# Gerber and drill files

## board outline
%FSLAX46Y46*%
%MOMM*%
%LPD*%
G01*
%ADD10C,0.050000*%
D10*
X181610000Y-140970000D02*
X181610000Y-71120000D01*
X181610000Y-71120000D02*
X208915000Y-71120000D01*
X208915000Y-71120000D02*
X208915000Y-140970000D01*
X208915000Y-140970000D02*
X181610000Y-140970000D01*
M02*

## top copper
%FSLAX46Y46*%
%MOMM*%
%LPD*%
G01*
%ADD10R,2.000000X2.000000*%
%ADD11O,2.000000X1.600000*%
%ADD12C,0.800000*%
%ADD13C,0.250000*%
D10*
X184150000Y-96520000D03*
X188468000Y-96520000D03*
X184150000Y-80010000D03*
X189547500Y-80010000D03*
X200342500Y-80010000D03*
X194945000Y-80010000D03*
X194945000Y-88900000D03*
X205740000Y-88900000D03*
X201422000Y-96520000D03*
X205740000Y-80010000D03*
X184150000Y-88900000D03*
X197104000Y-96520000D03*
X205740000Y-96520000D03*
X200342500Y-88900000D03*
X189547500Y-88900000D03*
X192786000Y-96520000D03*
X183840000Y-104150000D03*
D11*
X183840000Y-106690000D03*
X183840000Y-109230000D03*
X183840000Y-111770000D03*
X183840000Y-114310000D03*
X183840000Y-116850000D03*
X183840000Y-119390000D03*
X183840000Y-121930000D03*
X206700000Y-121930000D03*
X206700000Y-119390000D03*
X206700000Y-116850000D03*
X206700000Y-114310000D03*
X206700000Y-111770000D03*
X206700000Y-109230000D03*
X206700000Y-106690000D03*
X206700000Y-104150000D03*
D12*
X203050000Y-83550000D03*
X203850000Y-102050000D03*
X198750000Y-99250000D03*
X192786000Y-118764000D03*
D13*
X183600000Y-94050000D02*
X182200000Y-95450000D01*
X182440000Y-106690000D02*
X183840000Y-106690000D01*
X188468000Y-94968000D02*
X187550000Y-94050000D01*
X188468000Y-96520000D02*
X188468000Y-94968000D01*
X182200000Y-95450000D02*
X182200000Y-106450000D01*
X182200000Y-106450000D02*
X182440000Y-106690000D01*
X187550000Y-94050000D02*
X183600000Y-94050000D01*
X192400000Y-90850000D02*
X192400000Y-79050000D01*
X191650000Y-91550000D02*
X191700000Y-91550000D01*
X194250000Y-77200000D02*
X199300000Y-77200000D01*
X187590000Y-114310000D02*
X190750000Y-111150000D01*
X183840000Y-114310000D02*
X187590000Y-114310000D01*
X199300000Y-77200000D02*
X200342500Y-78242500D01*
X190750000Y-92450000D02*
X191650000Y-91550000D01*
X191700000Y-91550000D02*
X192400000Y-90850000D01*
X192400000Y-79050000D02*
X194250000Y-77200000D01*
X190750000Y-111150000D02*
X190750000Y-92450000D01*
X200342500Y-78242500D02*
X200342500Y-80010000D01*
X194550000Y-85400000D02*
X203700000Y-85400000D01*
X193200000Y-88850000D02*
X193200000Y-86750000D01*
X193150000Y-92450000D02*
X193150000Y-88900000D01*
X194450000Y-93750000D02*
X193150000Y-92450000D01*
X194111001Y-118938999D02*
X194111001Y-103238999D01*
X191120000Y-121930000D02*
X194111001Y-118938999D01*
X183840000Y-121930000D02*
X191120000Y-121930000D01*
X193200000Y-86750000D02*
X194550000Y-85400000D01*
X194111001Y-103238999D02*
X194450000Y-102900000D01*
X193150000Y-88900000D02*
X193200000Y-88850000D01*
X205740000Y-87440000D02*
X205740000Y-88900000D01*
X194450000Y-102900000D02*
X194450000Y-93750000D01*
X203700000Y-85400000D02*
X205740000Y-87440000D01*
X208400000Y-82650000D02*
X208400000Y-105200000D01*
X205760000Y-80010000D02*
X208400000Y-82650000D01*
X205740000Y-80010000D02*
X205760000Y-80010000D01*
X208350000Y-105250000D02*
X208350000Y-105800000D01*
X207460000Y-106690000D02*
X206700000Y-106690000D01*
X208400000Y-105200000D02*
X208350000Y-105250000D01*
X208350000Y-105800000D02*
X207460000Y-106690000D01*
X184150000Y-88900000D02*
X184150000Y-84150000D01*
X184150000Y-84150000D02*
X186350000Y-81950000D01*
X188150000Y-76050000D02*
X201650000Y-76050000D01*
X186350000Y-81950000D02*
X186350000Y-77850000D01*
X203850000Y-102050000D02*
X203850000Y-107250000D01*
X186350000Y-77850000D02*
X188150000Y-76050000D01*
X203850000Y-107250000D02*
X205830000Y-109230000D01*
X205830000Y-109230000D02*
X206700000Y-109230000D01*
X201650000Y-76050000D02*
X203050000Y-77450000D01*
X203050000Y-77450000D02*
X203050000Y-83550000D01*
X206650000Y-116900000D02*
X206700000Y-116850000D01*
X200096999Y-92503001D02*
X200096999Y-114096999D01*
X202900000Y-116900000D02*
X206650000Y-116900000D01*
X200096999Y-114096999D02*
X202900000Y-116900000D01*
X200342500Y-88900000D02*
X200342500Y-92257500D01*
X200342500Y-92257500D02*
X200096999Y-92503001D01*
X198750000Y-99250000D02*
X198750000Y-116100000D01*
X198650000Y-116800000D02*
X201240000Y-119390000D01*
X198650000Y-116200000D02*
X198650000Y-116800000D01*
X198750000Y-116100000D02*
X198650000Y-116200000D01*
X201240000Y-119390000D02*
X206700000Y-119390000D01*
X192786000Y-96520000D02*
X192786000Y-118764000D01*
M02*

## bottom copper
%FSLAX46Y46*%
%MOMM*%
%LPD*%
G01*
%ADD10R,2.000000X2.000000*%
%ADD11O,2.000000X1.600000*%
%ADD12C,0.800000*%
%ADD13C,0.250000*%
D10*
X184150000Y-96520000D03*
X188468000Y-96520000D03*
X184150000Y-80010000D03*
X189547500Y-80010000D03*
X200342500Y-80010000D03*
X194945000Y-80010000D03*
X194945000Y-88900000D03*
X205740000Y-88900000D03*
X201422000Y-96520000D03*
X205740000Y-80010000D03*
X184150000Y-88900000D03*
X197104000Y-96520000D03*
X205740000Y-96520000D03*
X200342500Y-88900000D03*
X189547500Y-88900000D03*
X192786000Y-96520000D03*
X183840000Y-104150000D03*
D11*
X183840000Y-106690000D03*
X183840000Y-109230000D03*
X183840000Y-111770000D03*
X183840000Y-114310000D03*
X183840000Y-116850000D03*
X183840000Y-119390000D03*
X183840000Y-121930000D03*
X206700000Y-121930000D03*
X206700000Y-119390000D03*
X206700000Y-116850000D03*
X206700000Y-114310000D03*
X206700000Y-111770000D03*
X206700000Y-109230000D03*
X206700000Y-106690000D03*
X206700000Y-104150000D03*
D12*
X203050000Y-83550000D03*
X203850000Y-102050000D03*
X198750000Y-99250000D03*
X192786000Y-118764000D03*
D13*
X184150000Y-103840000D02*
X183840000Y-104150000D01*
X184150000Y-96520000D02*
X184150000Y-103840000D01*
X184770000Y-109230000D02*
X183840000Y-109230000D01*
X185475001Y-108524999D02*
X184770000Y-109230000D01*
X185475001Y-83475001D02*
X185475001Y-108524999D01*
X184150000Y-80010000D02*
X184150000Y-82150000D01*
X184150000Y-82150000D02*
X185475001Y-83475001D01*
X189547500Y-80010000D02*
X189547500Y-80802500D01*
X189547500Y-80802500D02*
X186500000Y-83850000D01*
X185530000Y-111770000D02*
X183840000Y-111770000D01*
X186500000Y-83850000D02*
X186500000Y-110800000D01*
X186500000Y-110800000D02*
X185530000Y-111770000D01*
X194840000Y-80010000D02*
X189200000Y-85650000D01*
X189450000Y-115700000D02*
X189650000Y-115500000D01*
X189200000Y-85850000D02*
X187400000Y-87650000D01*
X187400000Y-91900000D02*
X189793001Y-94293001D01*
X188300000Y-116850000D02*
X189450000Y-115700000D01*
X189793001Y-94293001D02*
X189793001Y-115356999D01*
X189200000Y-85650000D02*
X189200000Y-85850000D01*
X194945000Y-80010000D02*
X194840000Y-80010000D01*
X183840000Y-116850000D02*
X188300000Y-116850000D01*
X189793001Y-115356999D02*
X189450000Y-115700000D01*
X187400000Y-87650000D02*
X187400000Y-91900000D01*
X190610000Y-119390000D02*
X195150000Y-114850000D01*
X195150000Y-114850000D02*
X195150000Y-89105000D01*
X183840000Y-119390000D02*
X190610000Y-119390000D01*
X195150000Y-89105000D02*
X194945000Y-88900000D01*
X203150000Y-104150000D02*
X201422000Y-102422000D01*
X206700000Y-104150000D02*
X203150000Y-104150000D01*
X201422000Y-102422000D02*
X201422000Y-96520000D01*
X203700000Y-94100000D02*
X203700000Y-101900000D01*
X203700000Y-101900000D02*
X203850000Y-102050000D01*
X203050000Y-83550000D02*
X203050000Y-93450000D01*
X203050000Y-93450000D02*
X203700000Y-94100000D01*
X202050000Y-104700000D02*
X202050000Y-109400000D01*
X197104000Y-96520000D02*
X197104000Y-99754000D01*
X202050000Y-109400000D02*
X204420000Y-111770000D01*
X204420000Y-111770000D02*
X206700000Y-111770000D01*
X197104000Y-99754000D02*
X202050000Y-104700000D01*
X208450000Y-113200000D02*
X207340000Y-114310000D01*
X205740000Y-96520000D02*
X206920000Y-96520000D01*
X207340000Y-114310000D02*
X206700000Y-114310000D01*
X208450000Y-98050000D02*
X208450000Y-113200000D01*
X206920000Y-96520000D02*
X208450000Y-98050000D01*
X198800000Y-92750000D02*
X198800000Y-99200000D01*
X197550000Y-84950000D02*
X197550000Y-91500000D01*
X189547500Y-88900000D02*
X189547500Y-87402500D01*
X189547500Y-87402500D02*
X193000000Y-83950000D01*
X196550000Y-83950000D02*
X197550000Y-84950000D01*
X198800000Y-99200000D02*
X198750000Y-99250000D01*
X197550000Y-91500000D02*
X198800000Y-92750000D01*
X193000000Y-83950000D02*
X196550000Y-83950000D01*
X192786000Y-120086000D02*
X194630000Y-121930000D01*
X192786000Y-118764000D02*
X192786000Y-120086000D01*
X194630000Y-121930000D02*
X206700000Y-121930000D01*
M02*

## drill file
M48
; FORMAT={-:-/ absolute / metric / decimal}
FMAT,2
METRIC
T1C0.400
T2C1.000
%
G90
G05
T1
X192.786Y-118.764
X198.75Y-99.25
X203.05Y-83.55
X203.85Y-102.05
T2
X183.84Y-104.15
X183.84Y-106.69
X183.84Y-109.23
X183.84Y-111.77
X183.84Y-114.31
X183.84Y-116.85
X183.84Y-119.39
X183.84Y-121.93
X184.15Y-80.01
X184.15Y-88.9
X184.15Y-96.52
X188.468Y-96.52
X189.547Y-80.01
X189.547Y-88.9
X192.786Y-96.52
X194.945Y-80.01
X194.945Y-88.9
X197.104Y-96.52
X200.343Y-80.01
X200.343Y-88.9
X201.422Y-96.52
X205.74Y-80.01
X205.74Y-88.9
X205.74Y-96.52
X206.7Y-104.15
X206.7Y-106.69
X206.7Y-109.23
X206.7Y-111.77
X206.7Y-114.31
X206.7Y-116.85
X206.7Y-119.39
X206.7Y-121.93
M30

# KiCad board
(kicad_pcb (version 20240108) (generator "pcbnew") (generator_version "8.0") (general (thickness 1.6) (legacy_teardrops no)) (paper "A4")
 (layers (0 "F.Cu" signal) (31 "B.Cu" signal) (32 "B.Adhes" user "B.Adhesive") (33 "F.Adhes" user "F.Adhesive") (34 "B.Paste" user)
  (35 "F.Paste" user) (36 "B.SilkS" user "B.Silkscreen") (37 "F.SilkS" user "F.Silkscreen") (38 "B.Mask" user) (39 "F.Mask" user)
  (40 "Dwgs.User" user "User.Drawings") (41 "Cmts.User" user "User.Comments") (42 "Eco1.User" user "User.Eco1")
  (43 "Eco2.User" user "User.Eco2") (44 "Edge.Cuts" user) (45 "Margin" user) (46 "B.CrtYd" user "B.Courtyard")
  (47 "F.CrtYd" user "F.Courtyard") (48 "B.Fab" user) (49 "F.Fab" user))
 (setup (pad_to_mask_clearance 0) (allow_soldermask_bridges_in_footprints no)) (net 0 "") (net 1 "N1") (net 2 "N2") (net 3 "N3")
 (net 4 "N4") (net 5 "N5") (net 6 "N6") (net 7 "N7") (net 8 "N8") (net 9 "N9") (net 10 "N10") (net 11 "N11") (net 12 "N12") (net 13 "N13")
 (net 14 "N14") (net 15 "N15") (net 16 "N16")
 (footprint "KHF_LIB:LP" (layer "F.Cu") (at 184.15 96.52)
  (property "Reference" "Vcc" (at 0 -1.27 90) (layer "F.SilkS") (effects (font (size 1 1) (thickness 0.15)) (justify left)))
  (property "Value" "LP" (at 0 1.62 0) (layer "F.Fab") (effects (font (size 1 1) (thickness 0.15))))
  (pad "1" thru_hole rect (at 0 0) (size 2 2) (drill 1) (layers "*.Cu" "*.Mask") (remove_unused_layers no) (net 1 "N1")))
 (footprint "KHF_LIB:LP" (layer "F.Cu") (at 188.468 96.52)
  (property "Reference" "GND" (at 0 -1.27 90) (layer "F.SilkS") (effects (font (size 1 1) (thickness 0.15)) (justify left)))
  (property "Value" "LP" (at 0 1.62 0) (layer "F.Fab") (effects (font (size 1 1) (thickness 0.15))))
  (pad "1" thru_hole rect (at 0 0) (size 2 2) (drill 1) (layers "*.Cu" "*.Mask") (remove_unused_layers no) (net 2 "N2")))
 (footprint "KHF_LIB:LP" (layer "F.Cu") (at 184.15 80.01)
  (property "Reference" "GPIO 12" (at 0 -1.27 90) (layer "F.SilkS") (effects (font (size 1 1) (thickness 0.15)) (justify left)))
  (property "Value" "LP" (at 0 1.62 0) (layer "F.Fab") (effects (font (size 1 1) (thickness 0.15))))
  (pad "1" thru_hole rect (at 0 0) (size 2 2) (drill 1) (layers "*.Cu" "*.Mask") (remove_unused_layers no) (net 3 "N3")))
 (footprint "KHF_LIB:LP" (layer "F.Cu") (at 189.5475 80.01)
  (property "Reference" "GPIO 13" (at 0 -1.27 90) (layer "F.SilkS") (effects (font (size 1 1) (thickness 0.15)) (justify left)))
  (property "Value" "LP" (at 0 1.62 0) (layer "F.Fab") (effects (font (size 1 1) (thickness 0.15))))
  (pad "1" thru_hole rect (at 0 0) (size 2 2) (drill 1) (layers "*.Cu" "*.Mask") (remove_unused_layers no) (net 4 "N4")))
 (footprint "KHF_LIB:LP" (layer "F.Cu") (at 200.3425 80.01)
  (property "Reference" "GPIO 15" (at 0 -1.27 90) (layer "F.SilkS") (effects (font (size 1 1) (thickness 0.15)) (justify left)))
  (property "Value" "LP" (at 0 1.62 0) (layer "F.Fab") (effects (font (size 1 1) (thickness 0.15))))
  (pad "1" thru_hole rect (at 0 0) (size 2 2) (drill 1) (layers "*.Cu" "*.Mask") (remove_unused_layers no) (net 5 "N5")))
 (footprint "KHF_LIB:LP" (layer "F.Cu") (at 194.945 80.01)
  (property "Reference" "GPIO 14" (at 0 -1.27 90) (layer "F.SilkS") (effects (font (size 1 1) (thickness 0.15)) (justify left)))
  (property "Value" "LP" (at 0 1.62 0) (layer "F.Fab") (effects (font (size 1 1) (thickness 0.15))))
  (pad "1" thru_hole rect (at 0 0) (size 2 2) (drill 1) (layers "*.Cu" "*.Mask") (remove_unused_layers no) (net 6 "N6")))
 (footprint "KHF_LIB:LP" (layer "F.Cu") (at 194.945 88.9)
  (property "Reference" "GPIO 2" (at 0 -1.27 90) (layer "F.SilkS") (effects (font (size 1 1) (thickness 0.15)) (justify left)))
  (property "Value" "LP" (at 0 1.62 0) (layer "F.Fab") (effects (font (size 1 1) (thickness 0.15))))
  (pad "1" thru_hole rect (at 0 0) (size 2 2) (drill 1) (layers "*.Cu" "*.Mask") (remove_unused_layers no) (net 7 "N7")))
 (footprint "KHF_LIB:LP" (layer "F.Cu") (at 205.74 88.9)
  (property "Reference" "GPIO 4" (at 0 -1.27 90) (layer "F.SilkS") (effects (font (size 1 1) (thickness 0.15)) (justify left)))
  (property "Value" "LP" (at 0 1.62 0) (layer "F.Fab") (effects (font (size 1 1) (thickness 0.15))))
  (pad "1" thru_hole rect (at 0 0) (size 2 2) (drill 1) (layers "*.Cu" "*.Mask") (remove_unused_layers no) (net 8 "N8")))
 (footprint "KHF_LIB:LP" (layer "F.Cu") (at 201.422 96.52)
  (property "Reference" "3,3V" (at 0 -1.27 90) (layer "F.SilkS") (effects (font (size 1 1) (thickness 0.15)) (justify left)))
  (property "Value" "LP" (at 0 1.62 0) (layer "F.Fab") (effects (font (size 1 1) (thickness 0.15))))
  (pad "1" thru_hole rect (at 0 0) (size 2 2) (drill 1) (layers "*.Cu" "*.Mask") (remove_unused_layers no) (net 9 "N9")))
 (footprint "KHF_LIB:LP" (layer "F.Cu") (at 205.74 80.01)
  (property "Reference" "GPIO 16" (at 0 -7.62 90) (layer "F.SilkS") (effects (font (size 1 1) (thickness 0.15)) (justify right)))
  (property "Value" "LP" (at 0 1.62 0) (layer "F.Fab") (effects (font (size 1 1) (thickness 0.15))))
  (pad "1" thru_hole rect (at 0 0) (size 2 2) (drill 1) (layers "*.Cu" "*.Mask") (remove_unused_layers no) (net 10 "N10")))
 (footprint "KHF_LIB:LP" (layer "F.Cu") (at 184.15 88.9)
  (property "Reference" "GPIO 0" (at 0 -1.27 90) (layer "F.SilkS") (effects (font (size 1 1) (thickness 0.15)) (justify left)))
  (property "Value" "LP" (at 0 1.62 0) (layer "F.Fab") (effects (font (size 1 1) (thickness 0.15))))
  (pad "1" thru_hole rect (at 0 0) (size 2 2) (drill 1) (layers "*.Cu" "*.Mask") (remove_unused_layers no) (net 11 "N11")))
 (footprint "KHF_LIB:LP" (layer "F.Cu") (at 197.104 96.52)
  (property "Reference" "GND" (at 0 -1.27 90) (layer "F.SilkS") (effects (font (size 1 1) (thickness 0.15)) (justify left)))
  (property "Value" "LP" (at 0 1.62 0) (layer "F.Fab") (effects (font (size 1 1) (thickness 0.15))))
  (pad "1" thru_hole rect (at 0 0) (size 2 2) (drill 1) (layers "*.Cu" "*.Mask") (remove_unused_layers no) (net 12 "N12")))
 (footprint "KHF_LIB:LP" (layer "F.Cu") (at 205.74 96.52)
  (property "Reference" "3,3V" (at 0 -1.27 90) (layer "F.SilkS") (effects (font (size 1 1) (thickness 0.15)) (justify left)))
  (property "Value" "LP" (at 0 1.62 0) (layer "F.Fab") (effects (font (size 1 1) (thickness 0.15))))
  (pad "1" thru_hole rect (at 0 0) (size 2 2) (drill 1) (layers "*.Cu" "*.Mask") (remove_unused_layers no) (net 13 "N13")))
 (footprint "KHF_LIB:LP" (layer "F.Cu") (at 200.3425 88.9)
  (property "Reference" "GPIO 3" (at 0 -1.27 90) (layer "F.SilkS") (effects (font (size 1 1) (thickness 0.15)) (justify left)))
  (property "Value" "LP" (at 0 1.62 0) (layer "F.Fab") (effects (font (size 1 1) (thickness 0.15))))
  (pad "1" thru_hole rect (at 0 0) (size 2 2) (drill 1) (layers "*.Cu" "*.Mask") (remove_unused_layers no) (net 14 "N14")))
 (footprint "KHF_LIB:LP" (layer "F.Cu") (at 189.5475 88.9)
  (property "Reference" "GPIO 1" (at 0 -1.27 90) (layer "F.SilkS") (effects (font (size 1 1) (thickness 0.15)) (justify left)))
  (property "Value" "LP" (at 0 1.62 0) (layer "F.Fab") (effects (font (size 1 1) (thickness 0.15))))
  (pad "1" thru_hole rect (at 0 0) (size 2 2) (drill 1) (layers "*.Cu" "*.Mask") (remove_unused_layers no) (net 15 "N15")))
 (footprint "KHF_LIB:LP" (layer "F.Cu") (at 192.786 96.52)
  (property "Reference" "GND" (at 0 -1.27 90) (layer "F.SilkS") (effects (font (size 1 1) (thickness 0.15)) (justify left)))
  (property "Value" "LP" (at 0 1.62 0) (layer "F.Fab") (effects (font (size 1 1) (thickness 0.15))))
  (pad "1" thru_hole rect (at 0 0) (size 2 2) (drill 1) (layers "*.Cu" "*.Mask") (remove_unused_layers no) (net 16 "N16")))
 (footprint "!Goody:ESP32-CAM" (layer "F.Cu") (at 195.27 118.16)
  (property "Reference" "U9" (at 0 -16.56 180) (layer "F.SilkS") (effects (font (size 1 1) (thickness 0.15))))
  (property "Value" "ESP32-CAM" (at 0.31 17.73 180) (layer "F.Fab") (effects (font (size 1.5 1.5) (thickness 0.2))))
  (pad "1" thru_hole rect (at -11.43 -14.01) (size 2 2) (drill 1) (layers "*.Cu" "*.Mask") (remove_unused_layers no) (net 1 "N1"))
  (pad "2" thru_hole oval (at -11.43 -11.47) (size 2 1.6) (drill 1) (layers "*.Cu" "*.Mask") (remove_unused_layers no) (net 2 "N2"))
  (pad "3" thru_hole oval (at -11.43 -8.93) (size 2 1.6) (drill 1) (layers "*.Cu" "*.Mask") (remove_unused_layers no) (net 3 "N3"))
  (pad "4" thru_hole oval (at -11.43 -6.39) (size 2 1.6) (drill 1) (layers "*.Cu" "*.Mask") (remove_unused_layers no) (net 4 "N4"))
  (pad "5" thru_hole oval (at -11.43 -3.85) (size 2 1.6) (drill 1) (layers "*.Cu" "*.Mask") (remove_unused_layers no) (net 5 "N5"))
  (pad "6" thru_hole oval (at -11.43 -1.31) (size 2 1.6) (drill 1) (layers "*.Cu" "*.Mask") (remove_unused_layers no) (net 6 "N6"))
  (pad "7" thru_hole oval (at -11.43 1.23) (size 2 1.6) (drill 1) (layers "*.Cu" "*.Mask") (remove_unused_layers no) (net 7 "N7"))
  (pad "8" thru_hole oval (at -11.43 3.77) (size 2 1.6) (drill 1) (layers "*.Cu" "*.Mask") (remove_unused_layers no) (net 8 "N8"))
  (pad "9" thru_hole oval (at 11.43 3.77) (size 2 1.6) (drill 1) (layers "*.Cu" "*.Mask") (remove_unused_layers no) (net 16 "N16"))
  (pad "10" thru_hole oval (at 11.43 1.23) (size 2 1.6) (drill 1) (layers "*.Cu" "*.Mask") (remove_unused_layers no) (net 15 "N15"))
  (pad "11" thru_hole oval (at 11.43 -1.31) (size 2 1.6) (drill 1) (layers "*.Cu" "*.Mask") (remove_unused_layers no) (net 14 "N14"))
  (pad "12" thru_hole oval (at 11.43 -3.85) (size 2 1.6) (drill 1) (layers "*.Cu" "*.Mask") (remove_unused_layers no) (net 13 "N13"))
  (pad "13" thru_hole oval (at 11.43 -6.39) (size 2 1.6) (drill 1) (layers "*.Cu" "*.Mask") (remove_unused_layers no) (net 12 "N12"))
  (pad "14" thru_hole oval (at 11.43 -8.93) (size 2 1.6) (drill 1) (layers "*.Cu" "*.Mask") (remove_unused_layers no) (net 11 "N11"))
  (pad "15" thru_hole oval (at 11.43 -11.47) (size 2 1.6) (drill 1) (layers "*.Cu" "*.Mask") (remove_unused_layers no) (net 10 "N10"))
  (pad "16" thru_hole oval (at 11.43 -14.01) (size 2 1.6) (drill 1) (layers "*.Cu" "*.Mask") (remove_unused_layers no) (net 9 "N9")))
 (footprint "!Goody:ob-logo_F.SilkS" (layer "F.Cu") (at 195.58 119.38)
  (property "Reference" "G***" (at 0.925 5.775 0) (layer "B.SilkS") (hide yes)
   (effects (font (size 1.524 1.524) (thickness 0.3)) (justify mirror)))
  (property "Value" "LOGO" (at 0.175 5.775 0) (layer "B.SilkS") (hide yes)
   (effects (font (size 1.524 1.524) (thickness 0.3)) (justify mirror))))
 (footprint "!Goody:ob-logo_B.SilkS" (layer "F.Cu") (at 201.93 135.89)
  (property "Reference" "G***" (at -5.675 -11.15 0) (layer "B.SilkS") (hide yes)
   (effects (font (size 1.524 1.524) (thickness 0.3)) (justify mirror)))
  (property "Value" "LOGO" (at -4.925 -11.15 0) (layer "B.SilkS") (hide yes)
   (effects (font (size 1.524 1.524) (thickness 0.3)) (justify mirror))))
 (gr_line (start 181.61 140.97) (end 181.61 71.12) (stroke (width 0.05) (type solid)) (layer "Edge.Cuts"))
 (gr_line (start 181.61 71.12) (end 208.915 71.12) (stroke (width 0.05) (type solid)) (layer "Edge.Cuts"))
 (gr_line (start 208.915 71.12) (end 208.915 140.97) (stroke (width 0.05) (type solid)) (layer "Edge.Cuts"))
 (gr_line (start 208.915 140.97) (end 181.61 140.97) (stroke (width 0.05) (type solid)) (layer "Edge.Cuts"))
 (segment (start 184.15 103.84) (end 183.84 104.15) (width 0.25) (layer "B.Cu") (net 1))
 (segment (start 184.15 96.52) (end 184.15 103.84) (width 0.25) (layer "B.Cu") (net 1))
 (segment (start 183.6 94.05) (end 182.2 95.45) (width 0.25) (layer "F.Cu") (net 2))
 (segment (start 182.44 106.69) (end 183.84 106.69) (width 0.25) (layer "F.Cu") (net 2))
 (segment (start 188.468 94.968) (end 187.55 94.05) (width 0.25) (layer "F.Cu") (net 2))
 (segment (start 188.468 96.52) (end 188.468 94.968) (width 0.25) (layer "F.Cu") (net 2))
 (segment (start 182.2 95.45) (end 182.2 106.45) (width 0.25) (layer "F.Cu") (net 2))
 (segment (start 182.2 106.45) (end 182.44 106.69) (width 0.25) (layer "F.Cu") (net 2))
 (segment (start 187.55 94.05) (end 183.6 94.05) (width 0.25) (layer "F.Cu") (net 2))
 (segment (start 184.77 109.23) (end 183.84 109.23) (width 0.25) (layer "B.Cu") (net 3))
 (segment (start 185.475001 108.524999) (end 184.77 109.23) (width 0.25) (layer "B.Cu") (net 3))
 (segment (start 185.475001 83.475001) (end 185.475001 108.524999) (width 0.25) (layer "B.Cu") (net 3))
 (segment (start 184.15 80.01) (end 184.15 82.15) (width 0.25) (layer "B.Cu") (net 3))
 (segment (start 184.15 82.15) (end 185.475001 83.475001) (width 0.25) (layer "B.Cu") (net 3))
 (segment (start 189.5475 80.01) (end 189.5475 80.8025) (width 0.25) (layer "B.Cu") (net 4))
 (segment (start 189.5475 80.8025) (end 186.5 83.85) (width 0.25) (layer "B.Cu") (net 4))
 (segment (start 185.53 111.77) (end 183.84 111.77) (width 0.25) (layer "B.Cu") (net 4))
 (segment (start 186.5 83.85) (end 186.5 110.8) (width 0.25) (layer "B.Cu") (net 4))
 (segment (start 186.5 110.8) (end 185.53 111.77) (width 0.25) (layer "B.Cu") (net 4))
 (segment (start 192.4 90.85) (end 192.4 79.05) (width 0.25) (layer "F.Cu") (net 5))
 (segment (start 191.65 91.55) (end 191.7 91.55) (width 0.25) (layer "F.Cu") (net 5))
 (segment (start 194.25 77.2) (end 199.3 77.2) (width 0.25) (layer "F.Cu") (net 5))
 (segment (start 187.59 114.31) (end 190.75 111.15) (width 0.25) (layer "F.Cu") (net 5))
 (segment (start 183.84 114.31) (end 187.59 114.31) (width 0.25) (layer "F.Cu") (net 5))
 (segment (start 199.3 77.2) (end 200.3425 78.2425) (width 0.25) (layer "F.Cu") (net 5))
 (segment (start 190.75 92.45) (end 191.65 91.55) (width 0.25) (layer "F.Cu") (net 5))
 (segment (start 191.7 91.55) (end 192.4 90.85) (width 0.25) (layer "F.Cu") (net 5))
 (segment (start 192.4 79.05) (end 194.25 77.2) (width 0.25) (layer "F.Cu") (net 5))
 (segment (start 190.75 111.15) (end 190.75 92.45) (width 0.25) (layer "F.Cu") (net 5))
 (segment (start 200.3425 78.2425) (end 200.3425 80.01) (width 0.25) (layer "F.Cu") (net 5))
 (segment (start 194.84 80.01) (end 189.2 85.65) (width 0.25) (layer "B.Cu") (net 6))
 (segment (start 189.45 115.7) (end 189.65 115.5) (width 0.25) (layer "B.Cu") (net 6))
 (segment (start 189.2 85.85) (end 187.4 87.65) (width 0.25) (layer "B.Cu") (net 6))
 (segment (start 187.4 91.9) (end 189.793001 94.293001) (width 0.25) (layer "B.Cu") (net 6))
 (segment (start 188.3 116.85) (end 189.45 115.7) (width 0.25) (layer "B.Cu") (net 6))
 (segment (start 189.793001 94.293001) (end 189.793001 115.356999) (width 0.25) (layer "B.Cu") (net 6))
 (segment (start 189.2 85.65) (end 189.2 85.85) (width 0.25) (layer "B.Cu") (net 6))
 (segment (start 194.945 80.01) (end 194.84 80.01) (width 0.25) (layer "B.Cu") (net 6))
 (segment (start 183.84 116.85) (end 188.3 116.85) (width 0.25) (layer "B.Cu") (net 6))
 (segment (start 189.793001 115.356999) (end 189.45 115.7) (width 0.25) (layer "B.Cu") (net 6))
 (segment (start 187.4 87.65) (end 187.4 91.9) (width 0.25) (layer "B.Cu") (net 6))
 (segment (start 190.61 119.39) (end 195.15 114.85) (width 0.25) (layer "B.Cu") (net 7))
 (segment (start 195.15 114.85) (end 195.15 89.105) (width 0.25) (layer "B.Cu") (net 7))
 (segment (start 183.84 119.39) (end 190.61 119.39) (width 0.25) (layer "B.Cu") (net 7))
 (segment (start 195.15 89.105) (end 194.945 88.9) (width 0.25) (layer "B.Cu") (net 7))
 (segment (start 194.55 85.4) (end 203.7 85.4) (width 0.25) (layer "F.Cu") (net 8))
 (segment (start 193.2 88.85) (end 193.2 86.75) (width 0.25) (layer "F.Cu") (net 8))
 (segment (start 193.15 92.45) (end 193.15 88.9) (width 0.25) (layer "F.Cu") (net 8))
 (segment (start 194.45 93.75) (end 193.15 92.45) (width 0.25) (layer "F.Cu") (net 8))
 (segment (start 194.111001 118.938999) (end 194.111001 103.238999) (width 0.25) (layer "F.Cu") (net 8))
 (segment (start 191.12 121.93) (end 194.111001 118.938999) (width 0.25) (layer "F.Cu") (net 8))
 (segment (start 183.84 121.93) (end 191.12 121.93) (width 0.25) (layer "F.Cu") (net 8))
 (segment (start 193.2 86.75) (end 194.55 85.4) (width 0.25) (layer "F.Cu") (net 8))
 (segment (start 194.111001 103.238999) (end 194.45 102.9) (width 0.25) (layer "F.Cu") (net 8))
 (segment (start 193.15 88.9) (end 193.2 88.85) (width 0.25) (layer "F.Cu") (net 8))
 (segment (start 205.74 87.44) (end 205.74 88.9) (width 0.25) (layer "F.Cu") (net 8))
 (segment (start 194.45 102.9) (end 194.45 93.75) (width 0.25) (layer "F.Cu") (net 8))
 (segment (start 203.7 85.4) (end 205.74 87.44) (width 0.25) (layer "F.Cu") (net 8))
 (segment (start 203.15 104.15) (end 201.422 102.422) (width 0.25) (layer "B.Cu") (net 9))
 (segment (start 206.7 104.15) (end 203.15 104.15) (width 0.25) (layer "B.Cu") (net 9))
 (segment (start 201.422 102.422) (end 201.422 96.52) (width 0.25) (layer "B.Cu") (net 9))
 (segment (start 208.4 82.65) (end 208.4 105.2) (width 0.25) (layer "F.Cu") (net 10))
 (segment (start 205.76 80.01) (end 208.4 82.65) (width 0.25) (layer "F.Cu") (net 10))
 (segment (start 205.74 80.01) (end 205.76 80.01) (width 0.25) (layer "F.Cu") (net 10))
 (segment (start 208.35 105.25) (end 208.35 105.8) (width 0.25) (layer "F.Cu") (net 10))
 (segment (start 207.46 106.69) (end 206.7 106.69) (width 0.25) (layer "F.Cu") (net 10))
 (segment (start 208.4 105.2) (end 208.35 105.25) (width 0.25) (layer "F.Cu") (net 10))
 (segment (start 208.35 105.8) (end 207.46 106.69) (width 0.25) (layer "F.Cu") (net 10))
 (segment (start 184.15 88.9) (end 184.15 84.15) (width 0.25) (layer "F.Cu") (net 11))
 (segment (start 184.15 84.15) (end 186.35 81.95) (width 0.25) (layer "F.Cu") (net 11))
 (segment (start 188.15 76.05) (end 201.65 76.05) (width 0.25) (layer "F.Cu") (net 11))
 (segment (start 186.35 81.95) (end 186.35 77.85) (width 0.25) (layer "F.Cu") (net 11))
 (segment (start 203.85 102.05) (end 203.85 107.25) (width 0.25) (layer "F.Cu") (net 11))
 (segment (start 186.35 77.85) (end 188.15 76.05) (width 0.25) (layer "F.Cu") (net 11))
 (segment (start 203.85 107.25) (end 205.83 109.23) (width 0.25) (layer "F.Cu") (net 11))
 (segment (start 205.83 109.23) (end 206.7 109.23) (width 0.25) (layer "F.Cu") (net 11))
 (segment (start 201.65 76.05) (end 203.05 77.45) (width 0.25) (layer "F.Cu") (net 11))
 (segment (start 203.05 77.45) (end 203.05 83.55) (width 0.25) (layer "F.Cu") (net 11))
 (via (at 203.05 83.55) (size 0.8) (drill 0.4) (layers "F.Cu" "B.Cu") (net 11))
 (via (at 203.85 102.05) (size 0.8) (drill 0.4) (layers "F.Cu" "B.Cu") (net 11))
 (segment (start 203.7 94.1) (end 203.7 101.9) (width 0.25) (layer "B.Cu") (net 11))
 (segment (start 203.7 101.9) (end 203.85 102.05) (width 0.25) (layer "B.Cu") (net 11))
 (segment (start 203.05 83.55) (end 203.05 93.45) (width 0.25) (layer "B.Cu") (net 11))
 (segment (start 203.05 93.45) (end 203.7 94.1) (width 0.25) (layer "B.Cu") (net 11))
 (segment (start 202.05 104.7) (end 202.05 109.4) (width 0.25) (layer "B.Cu") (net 12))
 (segment (start 197.104 96.52) (end 197.104 99.754) (width 0.25) (layer "B.Cu") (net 12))
 (segment (start 202.05 109.4) (end 204.42 111.77) (width 0.25) (layer "B.Cu") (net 12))
 (segment (start 204.42 111.77) (end 206.7 111.77) (width 0.25) (layer "B.Cu") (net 12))
 (segment (start 197.104 99.754) (end 202.05 104.7) (width 0.25) (layer "B.Cu") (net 12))
 (segment (start 208.45 113.2) (end 207.34 114.31) (width 0.25) (layer "B.Cu") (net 13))
 (segment (start 205.74 96.52) (end 206.92 96.52) (width 0.25) (layer "B.Cu") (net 13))
 (segment (start 207.34 114.31) (end 206.7 114.31) (width 0.25) (layer "B.Cu") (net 13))
 (segment (start 208.45 98.05) (end 208.45 113.2) (width 0.25) (layer "B.Cu") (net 13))
 (segment (start 206.92 96.52) (end 208.45 98.05) (width 0.25) (layer "B.Cu") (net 13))
 (segment (start 206.65 116.9) (end 206.7 116.85) (width 0.25) (layer "F.Cu") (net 14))
 (segment (start 200.096999 92.503001) (end 200.096999 114.096999) (width 0.25) (layer "F.Cu") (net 14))
 (segment (start 202.9 116.9) (end 206.65 116.9) (width 0.25) (layer "F.Cu") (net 14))
 (segment (start 200.096999 114.096999) (end 202.9 116.9) (width 0.25) (layer "F.Cu") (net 14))
 (segment (start 200.3425 88.9) (end 200.3425 92.2575) (width 0.25) (layer "F.Cu") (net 14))
 (segment (start 200.3425 92.2575) (end 200.096999 92.503001) (width 0.25) (layer "F.Cu") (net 14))
 (segment (start 198.75 99.25) (end 198.75 116.1) (width 0.25) (layer "F.Cu") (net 15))
 (segment (start 198.65 116.8) (end 201.24 119.39) (width 0.25) (layer "F.Cu") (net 15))
 (segment (start 198.65 116.2) (end 198.65 116.8) (width 0.25) (layer "F.Cu") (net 15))
 (segment (start 198.75 116.1) (end 198.65 116.2) (width 0.25) (layer "F.Cu") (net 15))
 (segment (start 201.24 119.39) (end 206.7 119.39) (width 0.25) (layer "F.Cu") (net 15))
 (via (at 198.75 99.25) (size 0.8) (drill 0.4) (layers "F.Cu" "B.Cu") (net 15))
 (segment (start 198.8 92.75) (end 198.8 99.2) (width 0.25) (layer "B.Cu") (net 15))
 (segment (start 197.55 84.95) (end 197.55 91.5) (width 0.25) (layer "B.Cu") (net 15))
 (segment (start 189.5475 88.9) (end 189.5475 87.4025) (width 0.25) (layer "B.Cu") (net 15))
 (segment (start 189.5475 87.4025) (end 193 83.95) (width 0.25) (layer "B.Cu") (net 15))
 (segment (start 196.55 83.95) (end 197.55 84.95) (width 0.25) (layer "B.Cu") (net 15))
 (segment (start 198.8 99.2) (end 198.75 99.25) (width 0.25) (layer "B.Cu") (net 15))
 (segment (start 197.55 91.5) (end 198.8 92.75) (width 0.25) (layer "B.Cu") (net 15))
 (segment (start 193 83.95) (end 196.55 83.95) (width 0.25) (layer "B.Cu") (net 15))
 (segment (start 192.786 96.52) (end 192.786 118.764) (width 0.25) (layer "F.Cu") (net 16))
 (via (at 192.786 118.764) (size 0.8) (drill 0.4) (layers "F.Cu" "B.Cu") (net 16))
 (segment (start 192.786 120.086) (end 194.63 121.93) (width 0.25) (layer "B.Cu") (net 16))
 (segment (start 192.786 118.764) (end 192.786 120.086) (width 0.25) (layer "B.Cu") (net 16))
 (segment (start 194.63 121.93) (end 206.7 121.93) (width 0.25) (layer "B.Cu") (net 16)))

